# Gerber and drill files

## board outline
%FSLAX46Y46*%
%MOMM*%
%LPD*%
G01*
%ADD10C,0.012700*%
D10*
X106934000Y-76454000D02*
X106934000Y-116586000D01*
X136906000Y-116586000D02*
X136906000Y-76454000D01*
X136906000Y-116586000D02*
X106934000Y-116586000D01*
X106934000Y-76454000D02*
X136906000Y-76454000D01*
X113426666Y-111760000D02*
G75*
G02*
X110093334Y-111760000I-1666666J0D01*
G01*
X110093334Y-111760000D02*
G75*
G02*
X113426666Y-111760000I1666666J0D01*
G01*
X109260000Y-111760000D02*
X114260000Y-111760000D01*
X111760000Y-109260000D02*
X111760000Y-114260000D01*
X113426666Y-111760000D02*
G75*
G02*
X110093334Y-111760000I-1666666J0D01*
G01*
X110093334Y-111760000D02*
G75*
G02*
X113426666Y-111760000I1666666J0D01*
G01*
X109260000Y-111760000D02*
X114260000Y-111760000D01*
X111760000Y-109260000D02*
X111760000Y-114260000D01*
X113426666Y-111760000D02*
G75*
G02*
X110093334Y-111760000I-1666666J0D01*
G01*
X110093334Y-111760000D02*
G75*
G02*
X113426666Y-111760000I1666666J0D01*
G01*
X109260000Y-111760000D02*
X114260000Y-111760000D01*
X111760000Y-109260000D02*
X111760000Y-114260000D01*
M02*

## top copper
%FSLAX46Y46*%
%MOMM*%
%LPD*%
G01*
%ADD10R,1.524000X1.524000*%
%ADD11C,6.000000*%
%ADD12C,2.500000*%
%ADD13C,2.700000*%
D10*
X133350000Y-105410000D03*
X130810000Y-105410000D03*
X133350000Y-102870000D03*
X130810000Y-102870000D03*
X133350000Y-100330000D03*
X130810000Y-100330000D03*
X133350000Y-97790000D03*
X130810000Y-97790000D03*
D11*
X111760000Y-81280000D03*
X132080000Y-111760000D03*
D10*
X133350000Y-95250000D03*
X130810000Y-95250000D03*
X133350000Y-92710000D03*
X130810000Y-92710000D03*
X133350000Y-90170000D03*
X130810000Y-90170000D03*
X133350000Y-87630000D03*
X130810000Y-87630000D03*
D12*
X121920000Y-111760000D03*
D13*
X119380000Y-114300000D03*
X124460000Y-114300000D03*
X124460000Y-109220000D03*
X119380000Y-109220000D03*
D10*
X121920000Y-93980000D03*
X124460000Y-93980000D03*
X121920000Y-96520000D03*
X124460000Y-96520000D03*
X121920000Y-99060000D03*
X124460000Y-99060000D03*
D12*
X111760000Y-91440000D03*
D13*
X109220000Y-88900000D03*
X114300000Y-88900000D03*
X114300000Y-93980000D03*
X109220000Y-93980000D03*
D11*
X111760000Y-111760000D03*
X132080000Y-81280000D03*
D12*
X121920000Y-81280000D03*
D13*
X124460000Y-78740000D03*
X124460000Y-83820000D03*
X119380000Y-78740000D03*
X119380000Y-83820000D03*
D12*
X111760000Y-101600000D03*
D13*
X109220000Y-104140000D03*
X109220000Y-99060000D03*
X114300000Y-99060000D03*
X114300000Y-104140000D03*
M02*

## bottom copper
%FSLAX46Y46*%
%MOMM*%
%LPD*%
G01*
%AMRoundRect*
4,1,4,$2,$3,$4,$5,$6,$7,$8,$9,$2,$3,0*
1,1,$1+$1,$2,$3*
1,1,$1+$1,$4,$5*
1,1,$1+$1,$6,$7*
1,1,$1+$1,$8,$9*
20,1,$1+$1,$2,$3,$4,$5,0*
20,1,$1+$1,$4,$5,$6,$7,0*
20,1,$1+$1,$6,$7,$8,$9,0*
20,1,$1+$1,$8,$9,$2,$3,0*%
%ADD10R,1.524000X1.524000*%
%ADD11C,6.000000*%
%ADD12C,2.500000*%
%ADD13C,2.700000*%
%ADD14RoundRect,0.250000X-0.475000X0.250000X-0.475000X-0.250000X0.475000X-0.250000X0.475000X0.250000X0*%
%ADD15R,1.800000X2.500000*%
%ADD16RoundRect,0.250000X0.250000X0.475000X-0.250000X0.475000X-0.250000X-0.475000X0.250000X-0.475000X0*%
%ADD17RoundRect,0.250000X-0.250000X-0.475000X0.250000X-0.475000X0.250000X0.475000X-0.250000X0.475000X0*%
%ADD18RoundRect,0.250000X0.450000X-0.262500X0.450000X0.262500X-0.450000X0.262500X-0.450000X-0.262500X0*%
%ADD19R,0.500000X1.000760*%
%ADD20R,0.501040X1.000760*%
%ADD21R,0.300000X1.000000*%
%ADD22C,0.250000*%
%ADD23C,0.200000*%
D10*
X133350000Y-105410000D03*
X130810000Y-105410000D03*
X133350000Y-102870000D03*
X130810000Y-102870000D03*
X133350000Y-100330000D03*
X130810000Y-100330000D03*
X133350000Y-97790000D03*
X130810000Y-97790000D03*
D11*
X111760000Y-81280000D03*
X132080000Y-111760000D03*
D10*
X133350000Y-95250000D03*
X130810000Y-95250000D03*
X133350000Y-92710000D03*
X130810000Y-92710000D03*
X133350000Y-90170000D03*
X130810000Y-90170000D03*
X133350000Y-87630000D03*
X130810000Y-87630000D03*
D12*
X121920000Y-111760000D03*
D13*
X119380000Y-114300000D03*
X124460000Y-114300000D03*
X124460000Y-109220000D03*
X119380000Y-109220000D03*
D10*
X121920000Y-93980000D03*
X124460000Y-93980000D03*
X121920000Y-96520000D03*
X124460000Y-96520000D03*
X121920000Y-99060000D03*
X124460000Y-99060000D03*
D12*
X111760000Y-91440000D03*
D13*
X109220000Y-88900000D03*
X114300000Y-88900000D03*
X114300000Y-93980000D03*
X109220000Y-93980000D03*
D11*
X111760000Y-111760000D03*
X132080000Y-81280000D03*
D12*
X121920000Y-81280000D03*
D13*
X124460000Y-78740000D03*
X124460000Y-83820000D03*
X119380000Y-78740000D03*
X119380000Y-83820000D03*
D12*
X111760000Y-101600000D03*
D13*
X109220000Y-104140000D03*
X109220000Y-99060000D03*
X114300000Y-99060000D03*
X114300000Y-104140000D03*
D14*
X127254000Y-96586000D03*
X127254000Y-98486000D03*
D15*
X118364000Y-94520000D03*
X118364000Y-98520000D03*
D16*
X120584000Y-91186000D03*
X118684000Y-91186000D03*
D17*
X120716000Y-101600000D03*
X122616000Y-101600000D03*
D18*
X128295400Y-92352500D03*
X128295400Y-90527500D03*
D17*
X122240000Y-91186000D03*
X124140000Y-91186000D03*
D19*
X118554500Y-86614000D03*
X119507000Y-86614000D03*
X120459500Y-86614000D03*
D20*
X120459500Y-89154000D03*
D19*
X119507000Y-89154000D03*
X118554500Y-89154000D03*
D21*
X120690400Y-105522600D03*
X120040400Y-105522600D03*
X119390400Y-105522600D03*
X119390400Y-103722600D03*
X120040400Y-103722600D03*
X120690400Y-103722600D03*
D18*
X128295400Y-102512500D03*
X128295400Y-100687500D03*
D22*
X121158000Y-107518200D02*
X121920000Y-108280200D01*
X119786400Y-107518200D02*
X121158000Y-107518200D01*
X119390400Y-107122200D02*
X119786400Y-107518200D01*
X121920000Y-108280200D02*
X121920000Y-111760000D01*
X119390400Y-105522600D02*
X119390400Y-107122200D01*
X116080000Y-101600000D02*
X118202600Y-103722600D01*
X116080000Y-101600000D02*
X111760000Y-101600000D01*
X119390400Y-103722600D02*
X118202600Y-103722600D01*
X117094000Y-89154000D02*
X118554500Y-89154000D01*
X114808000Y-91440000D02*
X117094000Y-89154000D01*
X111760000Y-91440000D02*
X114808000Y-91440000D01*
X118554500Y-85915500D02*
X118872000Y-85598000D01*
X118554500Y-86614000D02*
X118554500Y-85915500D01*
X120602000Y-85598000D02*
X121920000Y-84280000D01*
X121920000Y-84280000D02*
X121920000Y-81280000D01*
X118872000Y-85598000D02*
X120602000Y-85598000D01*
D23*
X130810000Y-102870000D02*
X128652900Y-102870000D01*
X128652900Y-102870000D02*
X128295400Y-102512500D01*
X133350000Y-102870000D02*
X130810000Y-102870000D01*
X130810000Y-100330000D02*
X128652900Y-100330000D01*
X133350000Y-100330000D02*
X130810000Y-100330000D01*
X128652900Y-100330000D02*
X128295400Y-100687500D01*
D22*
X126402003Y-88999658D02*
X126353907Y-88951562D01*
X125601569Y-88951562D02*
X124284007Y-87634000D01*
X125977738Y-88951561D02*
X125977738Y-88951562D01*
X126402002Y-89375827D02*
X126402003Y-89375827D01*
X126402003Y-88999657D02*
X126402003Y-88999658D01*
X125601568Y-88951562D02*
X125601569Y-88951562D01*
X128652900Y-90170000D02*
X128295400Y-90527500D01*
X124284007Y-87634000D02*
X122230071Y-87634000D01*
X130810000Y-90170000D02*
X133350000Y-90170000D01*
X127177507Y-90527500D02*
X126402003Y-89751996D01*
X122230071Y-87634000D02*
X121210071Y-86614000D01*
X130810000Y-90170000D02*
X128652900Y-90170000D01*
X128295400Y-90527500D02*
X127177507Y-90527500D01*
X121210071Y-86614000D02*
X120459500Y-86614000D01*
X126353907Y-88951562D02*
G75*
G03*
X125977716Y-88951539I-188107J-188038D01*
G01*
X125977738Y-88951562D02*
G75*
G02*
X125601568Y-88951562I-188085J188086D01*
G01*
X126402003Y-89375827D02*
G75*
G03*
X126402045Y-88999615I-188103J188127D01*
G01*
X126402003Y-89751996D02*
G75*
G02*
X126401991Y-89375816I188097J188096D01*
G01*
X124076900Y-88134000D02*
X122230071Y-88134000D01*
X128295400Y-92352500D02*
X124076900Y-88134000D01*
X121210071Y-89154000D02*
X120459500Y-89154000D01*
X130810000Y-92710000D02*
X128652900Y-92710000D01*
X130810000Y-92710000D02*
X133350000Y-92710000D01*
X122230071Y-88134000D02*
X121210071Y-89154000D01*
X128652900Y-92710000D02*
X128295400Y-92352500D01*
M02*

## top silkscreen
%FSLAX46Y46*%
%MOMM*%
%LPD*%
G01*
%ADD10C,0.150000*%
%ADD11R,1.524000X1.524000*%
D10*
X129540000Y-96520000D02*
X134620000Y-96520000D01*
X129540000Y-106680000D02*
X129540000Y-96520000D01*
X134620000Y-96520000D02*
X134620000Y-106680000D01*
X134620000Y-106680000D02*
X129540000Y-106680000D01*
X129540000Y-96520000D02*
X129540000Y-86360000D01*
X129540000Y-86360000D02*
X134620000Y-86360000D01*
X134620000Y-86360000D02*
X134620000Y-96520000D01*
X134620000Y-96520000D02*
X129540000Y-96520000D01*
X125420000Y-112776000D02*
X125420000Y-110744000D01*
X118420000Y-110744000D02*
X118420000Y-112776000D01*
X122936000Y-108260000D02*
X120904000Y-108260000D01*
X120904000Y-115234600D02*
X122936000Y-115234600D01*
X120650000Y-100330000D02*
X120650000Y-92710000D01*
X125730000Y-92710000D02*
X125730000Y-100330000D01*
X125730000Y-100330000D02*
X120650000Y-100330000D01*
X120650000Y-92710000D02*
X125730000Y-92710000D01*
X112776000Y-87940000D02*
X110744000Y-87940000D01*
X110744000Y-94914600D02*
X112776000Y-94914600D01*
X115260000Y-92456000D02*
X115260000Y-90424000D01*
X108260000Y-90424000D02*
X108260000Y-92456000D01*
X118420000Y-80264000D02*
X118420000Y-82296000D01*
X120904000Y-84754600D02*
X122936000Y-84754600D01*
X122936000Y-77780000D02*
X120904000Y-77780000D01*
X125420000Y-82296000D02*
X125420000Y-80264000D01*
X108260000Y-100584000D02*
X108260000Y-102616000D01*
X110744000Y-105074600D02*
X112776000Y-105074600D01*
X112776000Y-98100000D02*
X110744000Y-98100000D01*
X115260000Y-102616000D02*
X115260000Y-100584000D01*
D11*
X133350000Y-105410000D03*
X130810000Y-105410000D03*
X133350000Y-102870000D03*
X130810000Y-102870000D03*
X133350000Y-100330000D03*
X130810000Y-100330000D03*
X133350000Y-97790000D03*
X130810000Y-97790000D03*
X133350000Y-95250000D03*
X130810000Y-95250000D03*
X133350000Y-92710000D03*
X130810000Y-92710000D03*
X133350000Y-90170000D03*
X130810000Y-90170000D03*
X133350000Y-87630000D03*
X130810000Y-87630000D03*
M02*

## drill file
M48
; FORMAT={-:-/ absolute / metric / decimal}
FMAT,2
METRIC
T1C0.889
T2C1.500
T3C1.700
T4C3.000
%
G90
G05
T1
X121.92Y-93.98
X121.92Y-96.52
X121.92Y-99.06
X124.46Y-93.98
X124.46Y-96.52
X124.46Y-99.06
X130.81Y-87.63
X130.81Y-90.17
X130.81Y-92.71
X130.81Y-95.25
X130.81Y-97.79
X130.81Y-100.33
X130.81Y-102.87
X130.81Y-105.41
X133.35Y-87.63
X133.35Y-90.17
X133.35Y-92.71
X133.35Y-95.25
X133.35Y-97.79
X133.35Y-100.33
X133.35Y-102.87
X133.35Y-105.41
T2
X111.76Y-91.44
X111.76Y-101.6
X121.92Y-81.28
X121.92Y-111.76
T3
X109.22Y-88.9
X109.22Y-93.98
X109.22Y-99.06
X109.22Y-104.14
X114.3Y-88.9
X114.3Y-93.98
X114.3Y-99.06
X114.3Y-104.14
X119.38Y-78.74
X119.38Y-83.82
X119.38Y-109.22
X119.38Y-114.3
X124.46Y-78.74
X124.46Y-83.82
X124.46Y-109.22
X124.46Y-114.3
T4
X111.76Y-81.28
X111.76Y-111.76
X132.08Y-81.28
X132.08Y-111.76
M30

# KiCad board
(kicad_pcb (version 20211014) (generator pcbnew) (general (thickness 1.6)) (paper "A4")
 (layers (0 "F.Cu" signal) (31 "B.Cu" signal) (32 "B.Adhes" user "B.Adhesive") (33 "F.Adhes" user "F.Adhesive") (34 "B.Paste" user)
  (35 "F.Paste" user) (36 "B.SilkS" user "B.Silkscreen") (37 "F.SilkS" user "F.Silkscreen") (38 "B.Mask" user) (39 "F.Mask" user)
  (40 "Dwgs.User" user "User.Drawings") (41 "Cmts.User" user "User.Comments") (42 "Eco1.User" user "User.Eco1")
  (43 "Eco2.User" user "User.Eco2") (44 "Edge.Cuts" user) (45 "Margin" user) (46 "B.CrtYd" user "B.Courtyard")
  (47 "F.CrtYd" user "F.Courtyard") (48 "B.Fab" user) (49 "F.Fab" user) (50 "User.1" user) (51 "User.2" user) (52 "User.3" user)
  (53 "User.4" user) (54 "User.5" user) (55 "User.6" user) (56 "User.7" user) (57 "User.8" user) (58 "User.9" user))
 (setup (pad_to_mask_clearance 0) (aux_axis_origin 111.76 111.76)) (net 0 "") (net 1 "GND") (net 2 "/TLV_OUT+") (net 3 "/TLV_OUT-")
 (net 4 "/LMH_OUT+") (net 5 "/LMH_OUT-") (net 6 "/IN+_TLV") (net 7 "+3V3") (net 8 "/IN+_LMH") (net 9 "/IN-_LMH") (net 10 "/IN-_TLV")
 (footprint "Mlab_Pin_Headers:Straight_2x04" (layer "F.Cu") (at 132.08 101.6 180)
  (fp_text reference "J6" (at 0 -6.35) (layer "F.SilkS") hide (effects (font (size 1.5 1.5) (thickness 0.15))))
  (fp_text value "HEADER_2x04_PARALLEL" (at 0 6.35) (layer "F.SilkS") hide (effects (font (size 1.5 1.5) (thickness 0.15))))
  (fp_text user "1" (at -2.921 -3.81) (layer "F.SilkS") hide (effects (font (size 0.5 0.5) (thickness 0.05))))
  (fp_line (start 2.54 5.08) (end -2.54 5.08) (layer "F.SilkS") (width 0.15))
  (fp_line (start 2.54 -5.08) (end 2.54 5.08) (layer "F.SilkS") (width 0.15))
  (fp_line (start -2.54 5.08) (end -2.54 -5.08) (layer "F.SilkS") (width 0.15))
  (fp_line (start -2.54 -5.08) (end 2.54 -5.08) (layer "F.SilkS") (width 0.15))
  (pad "1" thru_hole rect (at -1.27 -3.81 180) (size 1.524 1.524) (drill 0.889) (layers *.Cu *.Mask "F.SilkS") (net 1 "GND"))
  (pad "2" thru_hole rect (at 1.27 -3.81 180) (size 1.524 1.524) (drill 0.889) (layers *.Cu *.Mask "F.SilkS") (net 1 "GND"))
  (pad "3" thru_hole rect (at -1.27 -1.27 180) (size 1.524 1.524) (drill 0.889) (layers *.Cu *.Mask "F.SilkS") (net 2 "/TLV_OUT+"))
  (pad "4" thru_hole rect (at 1.27 -1.27 180) (size 1.524 1.524) (drill 0.889) (layers *.Cu *.Mask "F.SilkS") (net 2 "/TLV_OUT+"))
  (pad "5" thru_hole rect (at -1.27 1.27 180) (size 1.524 1.524) (drill 0.889) (layers *.Cu *.Mask "F.SilkS") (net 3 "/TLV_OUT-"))
  (pad "6" thru_hole rect (at 1.27 1.27 180) (size 1.524 1.524) (drill 0.889) (layers *.Cu *.Mask "F.SilkS") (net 3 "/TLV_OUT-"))
  (pad "7" thru_hole rect (at -1.27 3.81 180) (size 1.524 1.524) (drill 0.889) (layers *.Cu *.Mask "F.SilkS") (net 1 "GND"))
  (pad "8" thru_hole rect (at 1.27 3.81 180) (size 1.524 1.524) (drill 0.889) (layers *.Cu *.Mask "F.SilkS") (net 1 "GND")))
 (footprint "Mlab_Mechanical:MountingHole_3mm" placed (layer "F.Cu") (at 111.76 81.28)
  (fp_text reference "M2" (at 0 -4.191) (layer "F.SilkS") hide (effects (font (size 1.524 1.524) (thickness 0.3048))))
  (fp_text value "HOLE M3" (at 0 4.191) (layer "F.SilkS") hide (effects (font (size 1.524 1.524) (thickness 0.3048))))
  (pad "1" thru_hole circle (at 0 0) (size 6 6) (drill 3) (layers *.Cu *.Mask) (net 1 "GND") (clearance 1) (zone_connect 2)))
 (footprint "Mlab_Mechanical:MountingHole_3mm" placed (layer "F.Cu") (at 132.08 111.76)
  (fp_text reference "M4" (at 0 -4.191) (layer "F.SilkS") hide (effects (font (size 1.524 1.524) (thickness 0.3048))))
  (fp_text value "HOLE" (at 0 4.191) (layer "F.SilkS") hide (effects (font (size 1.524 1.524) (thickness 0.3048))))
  (pad "1" thru_hole circle (at 0 0) (size 6 6) (drill 3) (layers *.Cu *.Mask) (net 1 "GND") (clearance 1) (zone_connect 2)))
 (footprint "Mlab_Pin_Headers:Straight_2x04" (layer "F.Cu") (at 132.08 91.44 180)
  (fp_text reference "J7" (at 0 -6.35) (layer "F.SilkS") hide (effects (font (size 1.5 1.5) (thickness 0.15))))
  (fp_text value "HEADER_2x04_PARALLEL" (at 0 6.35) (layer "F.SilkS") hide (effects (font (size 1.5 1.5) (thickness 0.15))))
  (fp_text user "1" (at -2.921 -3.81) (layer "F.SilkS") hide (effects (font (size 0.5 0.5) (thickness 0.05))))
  (fp_line (start 2.54 -5.08) (end 2.54 5.08) (layer "F.SilkS") (width 0.15))
  (fp_line (start 2.54 5.08) (end -2.54 5.08) (layer "F.SilkS") (width 0.15))
  (fp_line (start -2.54 5.08) (end -2.54 -5.08) (layer "F.SilkS") (width 0.15))
  (fp_line (start -2.54 -5.08) (end 2.54 -5.08) (layer "F.SilkS") (width 0.15))
  (pad "1" thru_hole rect (at -1.27 -3.81 180) (size 1.524 1.524) (drill 0.889) (layers *.Cu *.Mask "F.SilkS") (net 1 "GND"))
  (pad "2" thru_hole rect (at 1.27 -3.81 180) (size 1.524 1.524) (drill 0.889) (layers *.Cu *.Mask "F.SilkS") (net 1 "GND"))
  (pad "3" thru_hole rect (at -1.27 -1.27 180) (size 1.524 1.524) (drill 0.889) (layers *.Cu *.Mask "F.SilkS") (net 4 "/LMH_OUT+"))
  (pad "4" thru_hole rect (at 1.27 -1.27 180) (size 1.524 1.524) (drill 0.889) (layers *.Cu *.Mask "F.SilkS") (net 4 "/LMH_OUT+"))
  (pad "5" thru_hole rect (at -1.27 1.27 180) (size 1.524 1.524) (drill 0.889) (layers *.Cu *.Mask "F.SilkS") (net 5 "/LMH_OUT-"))
  (pad "6" thru_hole rect (at 1.27 1.27 180) (size 1.524 1.524) (drill 0.889) (layers *.Cu *.Mask "F.SilkS") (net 5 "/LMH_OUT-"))
  (pad "7" thru_hole rect (at -1.27 3.81 180) (size 1.524 1.524) (drill 0.889) (layers *.Cu *.Mask "F.SilkS") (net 1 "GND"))
  (pad "8" thru_hole rect (at 1.27 3.81 180) (size 1.524 1.524) (drill 0.889) (layers *.Cu *.Mask "F.SilkS") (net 1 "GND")))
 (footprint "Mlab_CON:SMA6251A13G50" (layer "F.Cu") (at 121.92 111.76)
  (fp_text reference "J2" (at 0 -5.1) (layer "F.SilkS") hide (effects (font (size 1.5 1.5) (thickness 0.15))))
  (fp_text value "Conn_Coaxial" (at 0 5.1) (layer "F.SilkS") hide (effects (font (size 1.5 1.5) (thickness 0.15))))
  (fp_line (start 3.5 1.016) (end 3.5 -1.016) (layer "F.SilkS") (width 0.15))
  (fp_line (start -3.5 -1.016) (end -3.5 1.016) (layer "F.SilkS") (width 0.15))
  (fp_line (start 1.016 -3.5) (end -1.016 -3.5) (layer "F.SilkS") (width 0.15))
  (fp_line (start -1.016 3.4746) (end 1.016 3.4746) (layer "F.SilkS") (width 0.15))
  (pad "1" thru_hole circle locked (at 0 0 180) (size 2.5 2.5) (drill 1.5) (layers *.Cu *.Mask) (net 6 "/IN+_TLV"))
  (pad "2" thru_hole circle locked (at -2.54 2.54 180) (size 2.7 2.7) (drill 1.7) (layers *.Cu *.Mask) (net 1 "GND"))
  (pad "2" thru_hole circle locked (at 2.54 2.54 180) (size 2.7 2.7) (drill 1.7) (layers *.Cu *.Mask) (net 1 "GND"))
  (pad "2" thru_hole circle locked (at 2.54 -2.54 180) (size 2.7 2.7) (drill 1.7) (layers *.Cu *.Mask) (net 1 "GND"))
  (pad "2" thru_hole circle locked (at -2.54 -2.54 180) (size 2.7 2.7) (drill 1.7) (layers *.Cu *.Mask) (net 1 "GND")))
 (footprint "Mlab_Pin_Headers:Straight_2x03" (layer "F.Cu") (at 123.19 96.52)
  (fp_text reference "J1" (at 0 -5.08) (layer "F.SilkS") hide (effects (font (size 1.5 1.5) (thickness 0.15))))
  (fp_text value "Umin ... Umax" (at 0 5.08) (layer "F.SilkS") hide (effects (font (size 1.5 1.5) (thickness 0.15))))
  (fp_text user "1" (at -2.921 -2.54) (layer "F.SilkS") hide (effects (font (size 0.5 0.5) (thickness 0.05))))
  (fp_line (start -2.54 3.81) (end -2.54 -3.81) (layer "F.SilkS") (width 0.15))
  (fp_line (start 2.54 -3.81) (end 2.54 3.81) (layer "F.SilkS") (width 0.15))
  (fp_line (start 2.54 3.81) (end -2.54 3.81) (layer "F.SilkS") (width 0.15))
  (fp_line (start -2.54 -3.81) (end 2.54 -3.81) (layer "F.SilkS") (width 0.15))
  (pad "1" thru_hole rect (at -1.27 -2.54) (size 1.524 1.524) (drill 0.889) (layers *.Cu *.Mask) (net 1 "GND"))
  (pad "2" thru_hole rect (at 1.27 -2.54) (size 1.524 1.524) (drill 0.889) (layers *.Cu *.Mask) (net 1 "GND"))
  (pad "3" thru_hole rect (at -1.27 0) (size 1.524 1.524) (drill 0.889) (layers *.Cu *.Mask) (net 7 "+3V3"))
  (pad "4" thru_hole rect (at 1.27 0) (size 1.524 1.524) (drill 0.889) (layers *.Cu *.Mask) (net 7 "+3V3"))
  (pad "5" thru_hole rect (at -1.27 2.54) (size 1.524 1.524) (drill 0.889) (layers *.Cu *.Mask) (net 1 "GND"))
  (pad "6" thru_hole rect (at 1.27 2.54) (size 1.524 1.524) (drill 0.889) (layers *.Cu *.Mask) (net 1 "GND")))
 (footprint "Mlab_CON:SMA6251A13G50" (layer "F.Cu") (at 111.76 91.44)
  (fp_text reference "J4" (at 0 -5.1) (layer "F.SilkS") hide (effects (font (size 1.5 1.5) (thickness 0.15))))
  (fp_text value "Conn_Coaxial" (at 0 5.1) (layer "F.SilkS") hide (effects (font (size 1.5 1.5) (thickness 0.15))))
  (fp_line (start 1.016 -3.5) (end -1.016 -3.5) (layer "F.SilkS") (width 0.15))
  (fp_line (start -1.016 3.4746) (end 1.016 3.4746) (layer "F.SilkS") (width 0.15))
  (fp_line (start 3.5 1.016) (end 3.5 -1.016) (layer "F.SilkS") (width 0.15))
  (fp_line (start -3.5 -1.016) (end -3.5 1.016) (layer "F.SilkS") (width 0.15))
  (pad "1" thru_hole circle locked (at 0 0 180) (size 2.5 2.5) (drill 1.5) (layers *.Cu *.Mask) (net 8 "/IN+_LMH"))
  (pad "2" thru_hole circle locked (at -2.54 -2.54 180) (size 2.7 2.7) (drill 1.7) (layers *.Cu *.Mask) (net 1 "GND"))
  (pad "2" thru_hole circle locked (at 2.54 -2.54 180) (size 2.7 2.7) (drill 1.7) (layers *.Cu *.Mask) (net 1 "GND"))
  (pad "2" thru_hole circle locked (at 2.54 2.54 180) (size 2.7 2.7) (drill 1.7) (layers *.Cu *.Mask) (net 1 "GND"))
  (pad "2" thru_hole circle locked (at -2.54 2.54 180) (size 2.7 2.7) (drill 1.7) (layers *.Cu *.Mask) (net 1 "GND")))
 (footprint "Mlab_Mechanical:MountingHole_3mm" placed (layer "F.Cu") (at 111.76 111.76)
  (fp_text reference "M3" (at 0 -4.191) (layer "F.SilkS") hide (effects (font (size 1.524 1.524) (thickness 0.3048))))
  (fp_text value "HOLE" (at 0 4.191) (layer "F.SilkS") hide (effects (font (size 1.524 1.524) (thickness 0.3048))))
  (pad "1" thru_hole circle (at 0 0) (size 6 6) (drill 3) (layers *.Cu *.Mask) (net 1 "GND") (clearance 1) (zone_connect 2)))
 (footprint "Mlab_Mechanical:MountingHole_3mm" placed (layer "F.Cu") (at 132.08 81.28)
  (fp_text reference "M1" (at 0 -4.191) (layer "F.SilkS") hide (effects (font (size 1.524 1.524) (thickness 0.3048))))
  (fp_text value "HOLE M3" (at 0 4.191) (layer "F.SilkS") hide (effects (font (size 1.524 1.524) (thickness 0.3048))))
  (pad "1" thru_hole circle (at 0 0) (size 6 6) (drill 3) (layers *.Cu *.Mask) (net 1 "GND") (clearance 1) (zone_connect 2)))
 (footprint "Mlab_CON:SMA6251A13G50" (layer "F.Cu") (at 121.92 81.28)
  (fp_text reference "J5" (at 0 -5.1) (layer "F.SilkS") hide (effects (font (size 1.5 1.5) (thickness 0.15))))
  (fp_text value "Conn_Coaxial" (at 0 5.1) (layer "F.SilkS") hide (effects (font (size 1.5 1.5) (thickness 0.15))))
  (fp_line (start -3.5 -1.016) (end -3.5 1.016) (layer "F.SilkS") (width 0.15))
  (fp_line (start -1.016 3.4746) (end 1.016 3.4746) (layer "F.SilkS") (width 0.15))
  (fp_line (start 1.016 -3.5) (end -1.016 -3.5) (layer "F.SilkS") (width 0.15))
  (fp_line (start 3.5 1.016) (end 3.5 -1.016) (layer "F.SilkS") (width 0.15))
  (pad "1" thru_hole circle locked (at 0 0 180) (size 2.5 2.5) (drill 1.5) (layers *.Cu *.Mask) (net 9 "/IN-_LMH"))
  (pad "2" thru_hole circle locked (at 2.54 -2.54 180) (size 2.7 2.7) (drill 1.7) (layers *.Cu *.Mask) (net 1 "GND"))
  (pad "2" thru_hole circle locked (at 2.54 2.54 180) (size 2.7 2.7) (drill 1.7) (layers *.Cu *.Mask) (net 1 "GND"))
  (pad "2" thru_hole circle locked (at -2.54 -2.54 180) (size 2.7 2.7) (drill 1.7) (layers *.Cu *.Mask) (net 1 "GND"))
  (pad "2" thru_hole circle locked (at -2.54 2.54 180) (size 2.7 2.7) (drill 1.7) (layers *.Cu *.Mask) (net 1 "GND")))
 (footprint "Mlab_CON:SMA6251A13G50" (layer "F.Cu") (at 111.76 101.6)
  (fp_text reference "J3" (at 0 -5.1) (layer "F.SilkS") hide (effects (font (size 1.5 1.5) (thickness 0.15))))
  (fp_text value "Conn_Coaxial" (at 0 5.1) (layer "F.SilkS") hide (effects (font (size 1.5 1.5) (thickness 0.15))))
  (fp_line (start -3.5 -1.016) (end -3.5 1.016) (layer "F.SilkS") (width 0.15))
  (fp_line (start -1.016 3.4746) (end 1.016 3.4746) (layer "F.SilkS") (width 0.15))
  (fp_line (start 1.016 -3.5) (end -1.016 -3.5) (layer "F.SilkS") (width 0.15))
  (fp_line (start 3.5 1.016) (end 3.5 -1.016) (layer "F.SilkS") (width 0.15))
  (pad "1" thru_hole circle locked (at 0 0 180) (size 2.5 2.5) (drill 1.5) (layers *.Cu *.Mask) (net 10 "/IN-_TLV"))
  (pad "2" thru_hole circle locked (at -2.54 2.54 180) (size 2.7 2.7) (drill 1.7) (layers *.Cu *.Mask) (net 1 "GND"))
  (pad "2" thru_hole circle locked (at -2.54 -2.54 180) (size 2.7 2.7) (drill 1.7) (layers *.Cu *.Mask) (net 1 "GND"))
  (pad "2" thru_hole circle locked (at 2.54 -2.54 180) (size 2.7 2.7) (drill 1.7) (layers *.Cu *.Mask) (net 1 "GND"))
  (pad "2" thru_hole circle locked (at 2.54 2.54 180) (size 2.7 2.7) (drill 1.7) (layers *.Cu *.Mask) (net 1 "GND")))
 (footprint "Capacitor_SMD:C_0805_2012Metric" (layer "B.Cu") (at 127.254 97.536 -90)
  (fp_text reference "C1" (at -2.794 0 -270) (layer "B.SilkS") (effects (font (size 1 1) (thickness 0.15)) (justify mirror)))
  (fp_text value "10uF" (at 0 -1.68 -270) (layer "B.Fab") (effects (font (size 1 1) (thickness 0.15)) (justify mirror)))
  (pad "1" smd roundrect (at -0.95 0 270) (size 1 1.45) (layers "B.Cu" "B.Paste" "B.Mask") (roundrect_rratio 0.25) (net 7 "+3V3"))
  (pad "2" smd roundrect (at 0.95 0 270) (size 1 1.45) (layers "B.Cu" "B.Paste" "B.Mask") (roundrect_rratio 0.25) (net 1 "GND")))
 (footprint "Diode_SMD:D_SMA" (layer "B.Cu") (at 118.364 96.52 -90)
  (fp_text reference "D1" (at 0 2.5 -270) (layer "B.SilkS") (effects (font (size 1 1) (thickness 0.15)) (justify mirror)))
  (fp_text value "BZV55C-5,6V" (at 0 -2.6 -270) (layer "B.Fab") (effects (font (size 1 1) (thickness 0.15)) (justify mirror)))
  (pad "1" smd rect (at -2 0 270) (size 2.5 1.8) (layers "B.Cu" "B.Paste" "B.Mask") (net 7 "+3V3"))
  (pad "2" smd rect (at 2 0 270) (size 2.5 1.8) (layers "B.Cu" "B.Paste" "B.Mask") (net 1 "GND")))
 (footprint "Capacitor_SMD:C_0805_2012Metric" (layer "B.Cu") (at 119.634 91.186 180)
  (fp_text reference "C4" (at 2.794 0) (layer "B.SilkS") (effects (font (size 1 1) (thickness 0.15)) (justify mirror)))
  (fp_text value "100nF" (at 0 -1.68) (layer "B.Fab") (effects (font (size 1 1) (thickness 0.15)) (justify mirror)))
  (pad "1" smd roundrect (at -0.95 0 180) (size 1 1.45) (layers "B.Cu" "B.Paste" "B.Mask") (roundrect_rratio 0.25) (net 7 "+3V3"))
  (pad "2" smd roundrect (at 0.95 0 180) (size 1 1.45) (layers "B.Cu" "B.Paste" "B.Mask") (roundrect_rratio 0.25) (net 1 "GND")))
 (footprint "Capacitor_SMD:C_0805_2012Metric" (layer "B.Cu") (at 121.666 101.6)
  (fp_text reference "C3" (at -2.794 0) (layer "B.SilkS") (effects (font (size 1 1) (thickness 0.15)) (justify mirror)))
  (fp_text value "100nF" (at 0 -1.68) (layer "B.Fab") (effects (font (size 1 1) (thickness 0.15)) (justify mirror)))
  (pad "1" smd roundrect (at -0.95 0) (size 1 1.45) (layers "B.Cu" "B.Paste" "B.Mask") (roundrect_rratio 0.25) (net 7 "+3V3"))
  (pad "2" smd roundrect (at 0.95 0) (size 1 1.45) (layers "B.Cu" "B.Paste" "B.Mask") (roundrect_rratio 0.25) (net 1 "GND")))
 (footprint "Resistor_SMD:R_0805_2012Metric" (layer "B.Cu") (at 128.2954 91.44 90)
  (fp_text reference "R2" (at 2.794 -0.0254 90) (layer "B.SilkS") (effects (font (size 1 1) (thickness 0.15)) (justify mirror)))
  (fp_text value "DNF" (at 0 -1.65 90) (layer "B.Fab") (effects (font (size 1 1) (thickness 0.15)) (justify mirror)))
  (pad "1" smd roundrect (at -0.9125 0 90) (size 1.025 1.4) (layers "B.Cu" "B.Paste" "B.Mask") (roundrect_rratio 0.243902)
   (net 4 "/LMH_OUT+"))
  (pad "2" smd roundrect (at 0.9125 0 90) (size 1.025 1.4) (layers "B.Cu" "B.Paste" "B.Mask") (roundrect_rratio 0.243902)
   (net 5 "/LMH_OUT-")))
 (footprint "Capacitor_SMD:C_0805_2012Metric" (layer "B.Cu") (at 123.19 91.186)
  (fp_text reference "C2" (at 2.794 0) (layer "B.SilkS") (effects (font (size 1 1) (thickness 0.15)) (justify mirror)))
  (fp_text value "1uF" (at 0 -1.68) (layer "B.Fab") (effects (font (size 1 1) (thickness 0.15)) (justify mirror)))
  (pad "1" smd roundrect (at -0.95 0) (size 1 1.45) (layers "B.Cu" "B.Paste" "B.Mask") (roundrect_rratio 0.25) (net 7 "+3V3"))
  (pad "2" smd roundrect (at 0.95 0) (size 1 1.45) (layers "B.Cu" "B.Paste" "B.Mask") (roundrect_rratio 0.25) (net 1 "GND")))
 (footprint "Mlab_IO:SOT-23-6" (layer "B.Cu") (at 119.507 87.884)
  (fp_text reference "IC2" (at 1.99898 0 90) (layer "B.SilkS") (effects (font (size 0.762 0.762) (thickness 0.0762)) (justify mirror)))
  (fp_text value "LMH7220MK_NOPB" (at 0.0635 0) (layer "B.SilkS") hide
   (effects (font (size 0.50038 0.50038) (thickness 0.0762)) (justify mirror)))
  (pad "1" smd rect locked (at -0.9525 -1.27) (size 0.5 1.00076) (layers "B.Cu" "B.Paste" "B.Mask") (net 9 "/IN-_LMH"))
  (pad "2" smd rect locked (at 0 -1.27) (size 0.5 1.00076) (layers "B.Cu" "B.Paste" "B.Mask") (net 1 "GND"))
  (pad "3" smd rect locked (at 0.9525 -1.27) (size 0.5 1.00076) (layers "B.Cu" "B.Paste" "B.Mask") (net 5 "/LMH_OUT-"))
  (pad "4" smd rect locked (at 0.9525 1.27) (size 0.50104 1.00076) (layers "B.Cu" "B.Paste" "B.Mask") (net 4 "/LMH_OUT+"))
  (pad "5" smd rect locked (at 0 1.27) (size 0.5 1.00076) (layers "B.Cu" "B.Paste" "B.Mask") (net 7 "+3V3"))
  (pad "6" smd rect locked (at -0.9525 1.27) (size 0.5 1.00076) (layers "B.Cu" "B.Paste" "B.Mask") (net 8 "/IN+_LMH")))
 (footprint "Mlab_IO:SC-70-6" (layer "B.Cu") (at 120.0404 104.6226 90)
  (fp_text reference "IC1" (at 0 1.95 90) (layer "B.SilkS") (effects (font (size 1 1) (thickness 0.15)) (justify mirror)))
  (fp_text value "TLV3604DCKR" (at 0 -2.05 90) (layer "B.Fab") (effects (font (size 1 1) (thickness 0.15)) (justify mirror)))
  (pad "1" smd rect locked (at -0.9 0.65 180) (size 0.3 1) (layers "B.Cu" "B.Paste" "B.Mask") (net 2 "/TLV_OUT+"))
  (pad "2" smd rect locked (at -0.9 0 180) (size 0.3 1) (layers "B.Cu" "B.Paste" "B.Mask") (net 1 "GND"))
  (pad "3" smd rect locked (at -0.9 -0.65 180) (size 0.3 1) (layers "B.Cu" "B.Paste" "B.Mask") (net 6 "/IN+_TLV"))
  (pad "4" smd rect locked (at 0.9 -0.65 180) (size 0.3 1) (layers "B.Cu" "B.Paste" "B.Mask") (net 10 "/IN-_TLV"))
  (pad "5" smd rect locked (at 0.9 0 180) (size 0.3 1) (layers "B.Cu" "B.Paste" "B.Mask") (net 7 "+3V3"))
  (pad "6" smd rect locked (at 0.9 0.65 180) (size 0.3 1) (layers "B.Cu" "B.Paste" "B.Mask") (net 3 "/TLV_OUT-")))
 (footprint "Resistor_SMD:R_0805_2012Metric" (layer "B.Cu") (at 128.2954 101.6 90)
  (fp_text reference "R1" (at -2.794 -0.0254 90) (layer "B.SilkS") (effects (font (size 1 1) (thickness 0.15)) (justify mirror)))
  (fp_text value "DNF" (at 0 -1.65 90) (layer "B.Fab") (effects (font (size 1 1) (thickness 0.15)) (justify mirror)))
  (pad "1" smd roundrect (at -0.9125 0 90) (size 1.025 1.4) (layers "B.Cu" "B.Paste" "B.Mask") (roundrect_rratio 0.243902)
   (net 2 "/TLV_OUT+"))
  (pad "2" smd roundrect (at 0.9125 0 90) (size 1.025 1.4) (layers "B.Cu" "B.Paste" "B.Mask") (roundrect_rratio 0.243902)
   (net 3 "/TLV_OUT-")))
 (gr_line (start 106.934 76.454) (end 106.934 116.586) (layer "Edge.Cuts") (width 0.0127))
 (gr_line (start 136.906 116.586) (end 136.906 76.454) (layer "Edge.Cuts") (width 0.0127))
 (gr_line (start 136.906 116.586) (end 106.934 116.586) (layer "Edge.Cuts") (width 0.0127))
 (gr_line (start 106.934 76.454) (end 136.906 76.454) (layer "Edge.Cuts") (width 0.0127))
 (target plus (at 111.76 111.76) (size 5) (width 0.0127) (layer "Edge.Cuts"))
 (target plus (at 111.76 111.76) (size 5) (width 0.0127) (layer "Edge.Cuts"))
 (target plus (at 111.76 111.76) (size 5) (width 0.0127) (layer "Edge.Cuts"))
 (segment (start 121.158 107.5182) (end 121.92 108.2802) (width 0.25) (layer "B.Cu") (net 6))
 (segment (start 119.7864 107.5182) (end 121.158 107.5182) (width 0.25) (layer "B.Cu") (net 6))
 (segment (start 119.3904 107.1222) (end 119.7864 107.5182) (width 0.25) (layer "B.Cu") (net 6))
 (segment (start 121.92 108.2802) (end 121.92 111.76) (width 0.25) (layer "B.Cu") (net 6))
 (segment (start 119.3904 105.5226) (end 119.3904 107.1222) (width 0.25) (layer "B.Cu") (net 6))
 (segment (start 116.08 101.6) (end 118.2026 103.7226) (width 0.25) (layer "B.Cu") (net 10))
 (segment (start 116.08 101.6) (end 111.76 101.6) (width 0.25) (layer "B.Cu") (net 10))
 (segment (start 119.3904 103.7226) (end 118.2026 103.7226) (width 0.25) (layer "B.Cu") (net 10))
 (segment (start 117.094 89.154) (end 118.5545 89.154) (width 0.25) (layer "B.Cu") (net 8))
 (segment (start 114.808 91.44) (end 117.094 89.154) (width 0.25) (layer "B.Cu") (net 8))
 (segment (start 111.76 91.44) (end 114.808 91.44) (width 0.25) (layer "B.Cu") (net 8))
 (segment (start 118.5545 85.9155) (end 118.872 85.598) (width 0.25) (layer "B.Cu") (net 9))
 (segment (start 118.5545 86.614) (end 118.5545 85.9155) (width 0.25) (layer "B.Cu") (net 9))
 (segment (start 120.602 85.598) (end 121.92 84.28) (width 0.25) (layer "B.Cu") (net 9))
 (segment (start 121.92 84.28) (end 121.92 81.28) (width 0.25) (layer "B.Cu") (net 9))
 (segment (start 118.872 85.598) (end 120.602 85.598) (width 0.25) (layer "B.Cu") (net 9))
 (segment (start 130.81 102.87) (end 128.6529 102.87) (width 0.2) (layer "B.Cu") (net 2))
 (segment (start 128.6529 102.87) (end 128.2954 102.5125) (width 0.2) (layer "B.Cu") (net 2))
 (segment (start 133.35 102.87) (end 130.81 102.87) (width 0.2) (layer "B.Cu") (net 2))
 (segment (start 130.81 100.33) (end 128.6529 100.33) (width 0.2) (layer "B.Cu") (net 3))
 (segment (start 133.35 100.33) (end 130.81 100.33) (width 0.2) (layer "B.Cu") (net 3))
 (segment (start 128.6529 100.33) (end 128.2954 100.6875) (width 0.2) (layer "B.Cu") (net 3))
 (segment (start 126.402003 88.999658) (end 126.353907 88.951562) (width 0.25) (layer "B.Cu") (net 5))
 (segment (start 125.601569 88.951562) (end 124.284007 87.634) (width 0.25) (layer "B.Cu") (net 5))
 (segment (start 125.977738 88.951561) (end 125.977738 88.951562) (width 0.25) (layer "B.Cu") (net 5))
 (segment (start 126.402002 89.375827) (end 126.402003 89.375827) (width 0.25) (layer "B.Cu") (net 5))
 (segment (start 126.402003 88.999657) (end 126.402003 88.999658) (width 0.25) (layer "B.Cu") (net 5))
 (segment (start 125.601568 88.951562) (end 125.601569 88.951562) (width 0.25) (layer "B.Cu") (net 5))
 (segment (start 128.6529 90.17) (end 128.2954 90.5275) (width 0.25) (layer "B.Cu") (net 5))
 (segment (start 124.284007 87.634) (end 122.230071 87.634) (width 0.25) (layer "B.Cu") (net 5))
 (segment (start 130.81 90.17) (end 133.35 90.17) (width 0.25) (layer "B.Cu") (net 5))
 (segment (start 127.177507 90.5275) (end 126.402003 89.751996) (width 0.25) (layer "B.Cu") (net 5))
 (segment (start 122.230071 87.634) (end 121.210071 86.614) (width 0.25) (layer "B.Cu") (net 5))
 (segment (start 130.81 90.17) (end 128.6529 90.17) (width 0.25) (layer "B.Cu") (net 5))
 (segment (start 128.2954 90.5275) (end 127.177507 90.5275) (width 0.25) (layer "B.Cu") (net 5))
 (segment (start 121.210071 86.614) (end 120.4595 86.614) (width 0.25) (layer "B.Cu") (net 5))
 (arc (start 126.353907 88.951562) (mid 126.165823 88.873654) (end 125.977738 88.951561) (width 0.25) (layer "B.Cu") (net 5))
 (arc (start 125.977738 88.951562) (mid 125.789653 89.029469) (end 125.601568 88.951562) (width 0.25) (layer "B.Cu") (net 5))
 (arc (start 126.402003 89.375827) (mid 126.47991 89.187742) (end 126.402003 88.999657) (width 0.25) (layer "B.Cu") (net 5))
 (arc (start 126.402003 89.751996) (mid 126.324095 89.563912) (end 126.402002 89.375827) (width 0.25) (layer "B.Cu") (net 5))
 (segment (start 124.0769 88.134) (end 122.230071 88.134) (width 0.25) (layer "B.Cu") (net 4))
 (segment (start 128.2954 92.3525) (end 124.0769 88.134) (width 0.25) (layer "B.Cu") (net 4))
 (segment (start 121.210071 89.154) (end 120.4595 89.154) (width 0.25) (layer "B.Cu") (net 4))
 (segment (start 130.81 92.71) (end 128.6529 92.71) (width 0.25) (layer "B.Cu") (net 4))
 (segment (start 130.81 92.71) (end 133.35 92.71) (width 0.25) (layer "B.Cu") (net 4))
 (segment (start 122.230071 88.134) (end 121.210071 89.154) (width 0.25) (layer "B.Cu") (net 4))
 (segment (start 128.6529 92.71) (end 128.2954 92.3525) (width 0.25) (layer "B.Cu") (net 4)))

